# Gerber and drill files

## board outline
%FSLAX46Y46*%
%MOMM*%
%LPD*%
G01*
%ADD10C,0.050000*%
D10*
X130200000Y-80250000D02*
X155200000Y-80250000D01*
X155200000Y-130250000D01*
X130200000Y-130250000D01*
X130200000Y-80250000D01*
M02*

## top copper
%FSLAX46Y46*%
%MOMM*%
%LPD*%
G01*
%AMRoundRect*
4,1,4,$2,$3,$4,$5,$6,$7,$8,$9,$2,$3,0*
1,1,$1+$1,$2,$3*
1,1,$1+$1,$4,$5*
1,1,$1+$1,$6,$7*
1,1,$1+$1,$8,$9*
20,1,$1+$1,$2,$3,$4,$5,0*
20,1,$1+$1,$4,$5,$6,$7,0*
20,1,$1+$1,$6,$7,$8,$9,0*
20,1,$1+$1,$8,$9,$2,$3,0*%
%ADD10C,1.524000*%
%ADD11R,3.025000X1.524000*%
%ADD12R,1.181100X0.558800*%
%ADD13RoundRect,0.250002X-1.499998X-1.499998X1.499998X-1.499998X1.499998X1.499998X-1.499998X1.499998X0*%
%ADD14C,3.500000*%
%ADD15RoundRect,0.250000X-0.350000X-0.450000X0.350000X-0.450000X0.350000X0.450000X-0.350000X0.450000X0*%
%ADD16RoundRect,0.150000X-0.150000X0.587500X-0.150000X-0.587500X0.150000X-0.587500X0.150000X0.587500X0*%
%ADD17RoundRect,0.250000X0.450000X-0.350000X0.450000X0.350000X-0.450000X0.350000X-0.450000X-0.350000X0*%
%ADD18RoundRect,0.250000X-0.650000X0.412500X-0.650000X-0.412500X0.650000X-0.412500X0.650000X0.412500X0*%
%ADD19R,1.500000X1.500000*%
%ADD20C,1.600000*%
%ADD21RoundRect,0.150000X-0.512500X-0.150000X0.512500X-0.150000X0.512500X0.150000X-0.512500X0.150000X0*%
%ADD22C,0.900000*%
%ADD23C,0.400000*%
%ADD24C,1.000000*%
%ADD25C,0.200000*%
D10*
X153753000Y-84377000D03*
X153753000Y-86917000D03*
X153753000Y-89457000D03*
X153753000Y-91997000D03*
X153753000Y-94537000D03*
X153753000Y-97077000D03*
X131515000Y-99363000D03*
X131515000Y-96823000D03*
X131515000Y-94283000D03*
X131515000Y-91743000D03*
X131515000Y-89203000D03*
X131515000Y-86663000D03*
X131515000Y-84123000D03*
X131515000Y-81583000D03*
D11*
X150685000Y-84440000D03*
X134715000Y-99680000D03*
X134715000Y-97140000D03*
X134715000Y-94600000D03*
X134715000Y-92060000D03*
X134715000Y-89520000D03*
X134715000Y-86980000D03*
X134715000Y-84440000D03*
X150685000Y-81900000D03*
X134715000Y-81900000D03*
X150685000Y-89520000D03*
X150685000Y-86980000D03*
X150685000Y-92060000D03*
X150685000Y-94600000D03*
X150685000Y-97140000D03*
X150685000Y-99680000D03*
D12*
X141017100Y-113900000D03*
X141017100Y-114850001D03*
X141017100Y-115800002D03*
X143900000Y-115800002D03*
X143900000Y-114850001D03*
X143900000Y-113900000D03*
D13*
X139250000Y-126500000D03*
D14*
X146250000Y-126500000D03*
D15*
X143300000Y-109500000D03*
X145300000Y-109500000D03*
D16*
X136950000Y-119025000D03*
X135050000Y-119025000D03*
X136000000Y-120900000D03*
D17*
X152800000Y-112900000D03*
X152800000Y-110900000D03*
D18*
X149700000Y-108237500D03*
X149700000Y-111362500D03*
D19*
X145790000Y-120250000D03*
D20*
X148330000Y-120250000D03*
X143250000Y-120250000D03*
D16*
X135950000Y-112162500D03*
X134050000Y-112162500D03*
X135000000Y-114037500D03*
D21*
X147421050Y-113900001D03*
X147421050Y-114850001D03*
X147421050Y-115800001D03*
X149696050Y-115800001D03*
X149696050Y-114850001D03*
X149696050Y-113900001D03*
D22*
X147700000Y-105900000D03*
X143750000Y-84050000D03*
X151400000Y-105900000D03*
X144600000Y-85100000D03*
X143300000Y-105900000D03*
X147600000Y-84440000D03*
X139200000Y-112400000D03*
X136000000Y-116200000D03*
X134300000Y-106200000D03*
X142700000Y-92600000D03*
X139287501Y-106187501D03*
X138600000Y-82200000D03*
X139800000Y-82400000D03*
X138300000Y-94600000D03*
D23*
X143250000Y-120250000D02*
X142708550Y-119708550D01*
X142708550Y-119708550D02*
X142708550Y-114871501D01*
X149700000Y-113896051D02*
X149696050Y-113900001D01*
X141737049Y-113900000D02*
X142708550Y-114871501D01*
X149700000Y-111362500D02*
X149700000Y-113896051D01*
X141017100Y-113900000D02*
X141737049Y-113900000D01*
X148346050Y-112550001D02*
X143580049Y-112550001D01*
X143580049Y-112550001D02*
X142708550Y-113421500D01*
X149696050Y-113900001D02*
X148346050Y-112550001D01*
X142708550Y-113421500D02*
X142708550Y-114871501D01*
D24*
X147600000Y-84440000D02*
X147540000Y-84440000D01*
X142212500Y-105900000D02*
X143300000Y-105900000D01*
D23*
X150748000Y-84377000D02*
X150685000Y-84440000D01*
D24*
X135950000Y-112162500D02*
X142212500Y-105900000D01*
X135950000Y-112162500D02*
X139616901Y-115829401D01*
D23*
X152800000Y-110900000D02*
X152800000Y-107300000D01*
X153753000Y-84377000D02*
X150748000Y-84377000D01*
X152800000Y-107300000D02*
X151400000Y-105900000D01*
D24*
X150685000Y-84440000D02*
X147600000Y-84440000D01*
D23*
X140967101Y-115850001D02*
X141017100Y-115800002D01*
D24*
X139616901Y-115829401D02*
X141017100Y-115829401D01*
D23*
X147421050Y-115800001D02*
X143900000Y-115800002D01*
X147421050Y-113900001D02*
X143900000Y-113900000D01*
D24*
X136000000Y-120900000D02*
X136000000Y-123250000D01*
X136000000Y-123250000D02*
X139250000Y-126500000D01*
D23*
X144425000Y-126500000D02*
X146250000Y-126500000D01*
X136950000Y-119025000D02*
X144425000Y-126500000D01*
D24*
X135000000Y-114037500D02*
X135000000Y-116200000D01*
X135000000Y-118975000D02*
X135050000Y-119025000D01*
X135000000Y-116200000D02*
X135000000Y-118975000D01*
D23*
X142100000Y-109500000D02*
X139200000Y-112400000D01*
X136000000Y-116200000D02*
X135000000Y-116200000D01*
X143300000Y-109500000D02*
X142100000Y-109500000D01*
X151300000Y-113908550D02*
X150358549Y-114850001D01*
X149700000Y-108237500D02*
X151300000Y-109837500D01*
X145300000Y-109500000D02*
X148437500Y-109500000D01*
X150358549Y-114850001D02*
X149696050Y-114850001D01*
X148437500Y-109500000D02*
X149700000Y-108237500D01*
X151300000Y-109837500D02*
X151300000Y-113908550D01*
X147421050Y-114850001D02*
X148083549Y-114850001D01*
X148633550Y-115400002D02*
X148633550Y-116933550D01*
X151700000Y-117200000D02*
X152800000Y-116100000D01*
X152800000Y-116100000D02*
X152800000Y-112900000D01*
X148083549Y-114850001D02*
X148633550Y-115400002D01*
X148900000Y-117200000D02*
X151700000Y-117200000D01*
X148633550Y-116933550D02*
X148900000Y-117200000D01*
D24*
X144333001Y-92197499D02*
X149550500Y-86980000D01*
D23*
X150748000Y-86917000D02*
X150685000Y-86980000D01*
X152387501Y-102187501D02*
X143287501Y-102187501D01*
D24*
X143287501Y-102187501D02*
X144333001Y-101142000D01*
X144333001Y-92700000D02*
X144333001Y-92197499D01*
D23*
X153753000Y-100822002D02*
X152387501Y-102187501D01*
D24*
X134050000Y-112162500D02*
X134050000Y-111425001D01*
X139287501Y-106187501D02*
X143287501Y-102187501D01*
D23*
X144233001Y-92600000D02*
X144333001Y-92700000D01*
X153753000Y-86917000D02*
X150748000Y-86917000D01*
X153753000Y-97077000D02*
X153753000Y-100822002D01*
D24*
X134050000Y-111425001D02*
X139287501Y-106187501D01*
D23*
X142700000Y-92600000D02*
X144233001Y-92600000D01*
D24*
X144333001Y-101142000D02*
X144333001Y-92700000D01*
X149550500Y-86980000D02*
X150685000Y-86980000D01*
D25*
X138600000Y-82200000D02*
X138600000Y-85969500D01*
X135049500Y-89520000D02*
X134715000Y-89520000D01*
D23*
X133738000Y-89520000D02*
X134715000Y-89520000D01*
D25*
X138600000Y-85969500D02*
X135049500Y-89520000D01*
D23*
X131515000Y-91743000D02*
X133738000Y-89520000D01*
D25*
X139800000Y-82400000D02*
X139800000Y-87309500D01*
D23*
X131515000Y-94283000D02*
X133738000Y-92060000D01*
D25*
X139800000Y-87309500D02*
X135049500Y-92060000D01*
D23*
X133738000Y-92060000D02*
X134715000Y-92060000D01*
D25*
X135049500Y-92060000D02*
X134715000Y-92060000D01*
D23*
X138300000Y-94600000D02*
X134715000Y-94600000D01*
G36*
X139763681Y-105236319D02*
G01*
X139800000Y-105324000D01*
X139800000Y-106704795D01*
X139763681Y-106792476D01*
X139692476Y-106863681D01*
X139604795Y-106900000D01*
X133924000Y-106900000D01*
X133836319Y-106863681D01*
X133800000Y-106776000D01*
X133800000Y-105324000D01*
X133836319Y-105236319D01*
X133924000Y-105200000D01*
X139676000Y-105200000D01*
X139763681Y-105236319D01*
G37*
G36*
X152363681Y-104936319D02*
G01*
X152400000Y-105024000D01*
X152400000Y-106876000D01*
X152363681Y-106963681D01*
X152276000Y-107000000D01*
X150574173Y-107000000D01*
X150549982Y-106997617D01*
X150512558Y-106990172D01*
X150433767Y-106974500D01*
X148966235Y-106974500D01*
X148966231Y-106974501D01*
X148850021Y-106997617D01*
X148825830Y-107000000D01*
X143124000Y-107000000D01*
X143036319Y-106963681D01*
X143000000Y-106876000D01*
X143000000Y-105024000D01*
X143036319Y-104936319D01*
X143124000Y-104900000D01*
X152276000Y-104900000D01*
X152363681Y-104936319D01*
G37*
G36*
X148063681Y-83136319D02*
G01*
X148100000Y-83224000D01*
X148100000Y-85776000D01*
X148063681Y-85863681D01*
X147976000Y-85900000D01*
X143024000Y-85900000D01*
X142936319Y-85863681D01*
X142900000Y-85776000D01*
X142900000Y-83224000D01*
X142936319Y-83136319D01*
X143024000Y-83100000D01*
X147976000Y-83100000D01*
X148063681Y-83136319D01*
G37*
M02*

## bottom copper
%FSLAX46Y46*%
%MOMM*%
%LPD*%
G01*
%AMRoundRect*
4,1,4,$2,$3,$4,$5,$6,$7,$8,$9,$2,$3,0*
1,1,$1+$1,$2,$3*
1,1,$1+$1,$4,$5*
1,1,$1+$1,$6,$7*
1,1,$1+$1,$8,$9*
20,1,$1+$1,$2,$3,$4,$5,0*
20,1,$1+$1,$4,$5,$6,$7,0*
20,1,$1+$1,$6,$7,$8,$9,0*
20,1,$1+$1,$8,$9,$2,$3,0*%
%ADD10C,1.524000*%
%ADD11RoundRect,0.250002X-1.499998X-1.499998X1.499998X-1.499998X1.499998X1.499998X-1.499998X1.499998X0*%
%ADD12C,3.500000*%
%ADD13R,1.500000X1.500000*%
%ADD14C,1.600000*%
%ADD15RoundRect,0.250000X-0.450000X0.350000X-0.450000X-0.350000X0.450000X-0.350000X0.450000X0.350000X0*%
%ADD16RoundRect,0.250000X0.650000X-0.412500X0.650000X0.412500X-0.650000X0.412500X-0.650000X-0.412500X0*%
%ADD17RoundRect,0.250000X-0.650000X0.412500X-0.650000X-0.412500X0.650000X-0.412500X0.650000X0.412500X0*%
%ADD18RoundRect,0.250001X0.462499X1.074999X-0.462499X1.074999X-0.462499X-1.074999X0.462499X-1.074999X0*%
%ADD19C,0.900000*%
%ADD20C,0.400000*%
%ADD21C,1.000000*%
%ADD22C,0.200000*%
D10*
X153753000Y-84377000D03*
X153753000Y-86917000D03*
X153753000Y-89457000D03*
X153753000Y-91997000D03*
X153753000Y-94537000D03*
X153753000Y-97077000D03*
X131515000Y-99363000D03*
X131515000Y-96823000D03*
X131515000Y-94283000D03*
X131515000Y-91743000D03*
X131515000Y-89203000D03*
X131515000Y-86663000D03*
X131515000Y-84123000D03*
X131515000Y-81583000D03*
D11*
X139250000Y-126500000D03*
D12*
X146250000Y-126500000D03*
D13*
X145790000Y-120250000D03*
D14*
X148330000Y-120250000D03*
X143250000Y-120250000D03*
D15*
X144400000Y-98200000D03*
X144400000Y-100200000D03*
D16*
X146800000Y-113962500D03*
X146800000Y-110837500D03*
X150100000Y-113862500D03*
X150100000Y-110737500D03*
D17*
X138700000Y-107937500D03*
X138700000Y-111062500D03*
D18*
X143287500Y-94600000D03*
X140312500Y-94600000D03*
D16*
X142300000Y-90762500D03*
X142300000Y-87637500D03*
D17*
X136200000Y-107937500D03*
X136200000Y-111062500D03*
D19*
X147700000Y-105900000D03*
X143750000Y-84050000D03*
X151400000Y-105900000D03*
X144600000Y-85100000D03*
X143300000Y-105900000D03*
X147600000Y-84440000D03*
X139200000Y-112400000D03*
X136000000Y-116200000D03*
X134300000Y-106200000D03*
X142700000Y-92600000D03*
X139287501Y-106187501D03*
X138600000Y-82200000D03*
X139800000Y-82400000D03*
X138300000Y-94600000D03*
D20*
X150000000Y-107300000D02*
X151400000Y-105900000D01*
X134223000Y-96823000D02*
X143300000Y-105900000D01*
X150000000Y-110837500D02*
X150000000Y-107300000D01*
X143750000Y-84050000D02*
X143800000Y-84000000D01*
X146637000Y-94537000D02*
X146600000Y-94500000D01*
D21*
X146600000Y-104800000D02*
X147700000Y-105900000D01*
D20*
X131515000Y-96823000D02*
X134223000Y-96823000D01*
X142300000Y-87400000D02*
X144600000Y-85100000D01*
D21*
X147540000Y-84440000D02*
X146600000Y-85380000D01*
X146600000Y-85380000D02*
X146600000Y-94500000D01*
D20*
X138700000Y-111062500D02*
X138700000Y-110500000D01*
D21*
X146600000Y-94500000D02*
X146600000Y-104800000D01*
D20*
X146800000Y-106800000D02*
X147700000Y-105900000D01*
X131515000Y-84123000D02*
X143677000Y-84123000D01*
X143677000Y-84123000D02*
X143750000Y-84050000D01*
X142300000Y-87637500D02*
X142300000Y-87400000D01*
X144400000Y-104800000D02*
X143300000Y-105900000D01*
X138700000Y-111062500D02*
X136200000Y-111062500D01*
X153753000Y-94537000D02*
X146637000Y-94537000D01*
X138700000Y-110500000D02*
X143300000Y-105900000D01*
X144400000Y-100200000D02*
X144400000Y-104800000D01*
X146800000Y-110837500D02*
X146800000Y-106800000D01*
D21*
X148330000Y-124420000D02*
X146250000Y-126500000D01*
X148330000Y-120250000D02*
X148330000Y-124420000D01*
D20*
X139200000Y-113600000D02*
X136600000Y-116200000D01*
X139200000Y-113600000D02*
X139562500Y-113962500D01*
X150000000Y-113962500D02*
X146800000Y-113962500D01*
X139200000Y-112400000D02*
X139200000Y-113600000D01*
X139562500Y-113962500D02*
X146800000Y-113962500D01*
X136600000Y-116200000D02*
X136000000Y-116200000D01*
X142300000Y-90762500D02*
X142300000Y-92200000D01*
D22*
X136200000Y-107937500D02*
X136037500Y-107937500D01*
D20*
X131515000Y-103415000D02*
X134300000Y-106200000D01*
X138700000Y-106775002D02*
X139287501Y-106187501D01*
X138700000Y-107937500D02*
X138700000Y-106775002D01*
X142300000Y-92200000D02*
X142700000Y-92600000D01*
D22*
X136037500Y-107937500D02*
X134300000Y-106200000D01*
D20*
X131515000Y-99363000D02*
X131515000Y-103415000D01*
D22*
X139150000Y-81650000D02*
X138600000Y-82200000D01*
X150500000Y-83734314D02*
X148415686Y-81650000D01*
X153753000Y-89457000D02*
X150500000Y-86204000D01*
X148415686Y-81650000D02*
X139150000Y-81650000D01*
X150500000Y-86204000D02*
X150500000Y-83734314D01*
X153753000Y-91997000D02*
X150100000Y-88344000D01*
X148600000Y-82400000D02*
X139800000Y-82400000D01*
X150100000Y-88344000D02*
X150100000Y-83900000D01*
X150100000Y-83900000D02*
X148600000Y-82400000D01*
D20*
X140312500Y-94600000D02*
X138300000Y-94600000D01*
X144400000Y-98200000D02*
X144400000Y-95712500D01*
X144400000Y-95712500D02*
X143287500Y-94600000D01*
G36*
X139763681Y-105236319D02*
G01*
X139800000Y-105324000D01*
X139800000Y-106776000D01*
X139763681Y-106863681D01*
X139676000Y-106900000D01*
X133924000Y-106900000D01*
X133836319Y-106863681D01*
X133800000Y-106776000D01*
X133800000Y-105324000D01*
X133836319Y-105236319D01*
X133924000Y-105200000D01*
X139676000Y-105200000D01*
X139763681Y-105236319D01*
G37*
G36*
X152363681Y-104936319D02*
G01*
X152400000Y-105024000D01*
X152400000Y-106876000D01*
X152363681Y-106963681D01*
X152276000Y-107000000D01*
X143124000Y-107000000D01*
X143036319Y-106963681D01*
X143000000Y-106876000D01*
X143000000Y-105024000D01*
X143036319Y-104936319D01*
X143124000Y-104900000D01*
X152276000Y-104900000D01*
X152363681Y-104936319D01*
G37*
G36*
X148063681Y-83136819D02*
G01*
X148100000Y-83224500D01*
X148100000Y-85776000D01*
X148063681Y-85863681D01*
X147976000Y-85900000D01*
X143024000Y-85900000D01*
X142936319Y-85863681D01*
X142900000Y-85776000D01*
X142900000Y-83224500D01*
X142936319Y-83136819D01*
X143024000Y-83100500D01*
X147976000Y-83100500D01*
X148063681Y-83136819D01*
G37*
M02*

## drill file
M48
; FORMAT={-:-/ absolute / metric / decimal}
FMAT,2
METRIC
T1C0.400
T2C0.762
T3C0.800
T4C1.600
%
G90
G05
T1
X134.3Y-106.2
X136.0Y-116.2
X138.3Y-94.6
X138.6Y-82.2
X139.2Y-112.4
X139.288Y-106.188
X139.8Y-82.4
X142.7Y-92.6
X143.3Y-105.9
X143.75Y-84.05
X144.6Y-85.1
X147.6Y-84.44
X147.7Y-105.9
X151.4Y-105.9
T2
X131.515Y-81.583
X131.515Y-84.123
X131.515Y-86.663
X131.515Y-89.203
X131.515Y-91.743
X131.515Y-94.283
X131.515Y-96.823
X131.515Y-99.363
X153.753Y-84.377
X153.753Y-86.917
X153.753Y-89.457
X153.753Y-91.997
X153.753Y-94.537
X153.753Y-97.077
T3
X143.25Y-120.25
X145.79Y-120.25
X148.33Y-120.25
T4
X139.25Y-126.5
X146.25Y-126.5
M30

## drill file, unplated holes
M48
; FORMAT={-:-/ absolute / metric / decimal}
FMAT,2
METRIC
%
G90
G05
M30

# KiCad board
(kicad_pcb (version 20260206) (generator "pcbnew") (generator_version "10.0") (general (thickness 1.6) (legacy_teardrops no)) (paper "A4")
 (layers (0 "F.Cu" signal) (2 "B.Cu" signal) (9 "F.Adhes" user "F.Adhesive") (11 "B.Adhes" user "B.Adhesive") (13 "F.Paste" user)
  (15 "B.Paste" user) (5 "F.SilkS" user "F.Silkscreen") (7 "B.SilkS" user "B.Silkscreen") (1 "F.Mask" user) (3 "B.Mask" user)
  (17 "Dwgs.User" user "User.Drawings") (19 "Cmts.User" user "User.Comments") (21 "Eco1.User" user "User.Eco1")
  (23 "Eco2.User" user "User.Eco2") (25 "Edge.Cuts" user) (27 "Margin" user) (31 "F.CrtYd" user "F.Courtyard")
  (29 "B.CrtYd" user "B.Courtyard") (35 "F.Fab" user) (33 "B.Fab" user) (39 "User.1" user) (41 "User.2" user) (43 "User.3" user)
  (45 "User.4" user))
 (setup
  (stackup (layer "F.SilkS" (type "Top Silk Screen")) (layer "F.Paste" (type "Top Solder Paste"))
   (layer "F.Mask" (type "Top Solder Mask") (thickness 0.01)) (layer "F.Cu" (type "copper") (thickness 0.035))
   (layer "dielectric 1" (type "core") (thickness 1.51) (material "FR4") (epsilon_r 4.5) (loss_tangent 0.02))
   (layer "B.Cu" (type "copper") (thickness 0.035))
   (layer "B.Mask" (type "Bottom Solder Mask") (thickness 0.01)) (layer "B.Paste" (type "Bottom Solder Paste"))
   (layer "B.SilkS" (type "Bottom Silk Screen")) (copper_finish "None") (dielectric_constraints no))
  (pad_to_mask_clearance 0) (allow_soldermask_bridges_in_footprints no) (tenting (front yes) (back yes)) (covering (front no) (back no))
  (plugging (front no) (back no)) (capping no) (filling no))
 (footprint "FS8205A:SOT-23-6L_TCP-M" (layer "F.Cu") (at 142.45855 114.850001)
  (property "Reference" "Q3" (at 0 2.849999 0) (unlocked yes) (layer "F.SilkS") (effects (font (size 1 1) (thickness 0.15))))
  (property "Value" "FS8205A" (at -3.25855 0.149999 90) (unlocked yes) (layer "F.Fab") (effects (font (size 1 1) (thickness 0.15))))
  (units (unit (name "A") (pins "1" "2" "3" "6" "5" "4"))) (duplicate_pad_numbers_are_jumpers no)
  (pad "1" smd rect (at -1.44145 -0.950001) (size 1.1811 0.5588) (layers "F.Cu" "F.Mask" "F.Paste") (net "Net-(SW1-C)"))
  (pad "2" smd rect (at -1.44145 0) (size 1.1811 0.5588) (layers "F.Cu" "F.Mask" "F.Paste") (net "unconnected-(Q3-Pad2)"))
  (pad "3" smd rect (at -1.44145 0.950001) (size 1.1811 0.5588) (layers "F.Cu" "F.Mask" "F.Paste") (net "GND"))
  (pad "4" smd rect (at 1.44145 0.950001) (size 1.1811 0.5588) (layers "F.Cu" "F.Mask" "F.Paste") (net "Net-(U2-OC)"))
  (pad "5" smd rect (at 1.44145 0) (size 1.1811 0.5588) (layers "F.Cu" "F.Mask" "F.Paste") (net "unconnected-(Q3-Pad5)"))
  (pad "6" smd rect (at 1.44145 -0.950001) (size 1.1811 0.5588) (layers "F.Cu" "F.Mask" "F.Paste") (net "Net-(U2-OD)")))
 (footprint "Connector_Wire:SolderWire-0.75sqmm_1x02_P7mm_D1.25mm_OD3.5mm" (layer "F.Cu") (at 139.25 126.5)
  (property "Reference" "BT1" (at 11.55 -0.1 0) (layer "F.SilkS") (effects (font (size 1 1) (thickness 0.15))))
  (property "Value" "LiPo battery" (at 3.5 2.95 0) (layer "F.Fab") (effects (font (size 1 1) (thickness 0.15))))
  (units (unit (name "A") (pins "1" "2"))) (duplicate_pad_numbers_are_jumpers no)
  (pad "1" thru_hole roundrect (at 0 0) (size 3.5 3.5) (drill 1.6) (layers "*.Cu" "*.Mask") (remove_unused_layers no)
   (roundrect_rratio 0.071429) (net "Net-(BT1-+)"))
  (pad "2" thru_hole circle (at 7 0) (size 3.5 3.5) (drill 1.6) (layers "*.Cu" "*.Mask") (remove_unused_layers no) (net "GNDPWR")))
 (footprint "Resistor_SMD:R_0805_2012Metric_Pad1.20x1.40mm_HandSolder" (layer "F.Cu") (at 144.3 109.5)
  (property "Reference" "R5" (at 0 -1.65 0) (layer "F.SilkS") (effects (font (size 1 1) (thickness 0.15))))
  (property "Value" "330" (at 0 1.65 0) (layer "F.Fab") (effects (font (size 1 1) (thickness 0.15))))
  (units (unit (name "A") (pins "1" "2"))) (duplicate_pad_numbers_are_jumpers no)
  (pad "1" smd roundrect (at -1 0) (size 1.2 1.4) (layers "F.Cu" "F.Mask" "F.Paste") (roundrect_rratio 0.208333) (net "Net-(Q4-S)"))
  (pad "2" smd roundrect (at 1 0) (size 1.2 1.4) (layers "F.Cu" "F.Mask" "F.Paste") (roundrect_rratio 0.208333) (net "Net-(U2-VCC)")))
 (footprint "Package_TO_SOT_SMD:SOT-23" (layer "F.Cu") (at 136 119.9625 -90)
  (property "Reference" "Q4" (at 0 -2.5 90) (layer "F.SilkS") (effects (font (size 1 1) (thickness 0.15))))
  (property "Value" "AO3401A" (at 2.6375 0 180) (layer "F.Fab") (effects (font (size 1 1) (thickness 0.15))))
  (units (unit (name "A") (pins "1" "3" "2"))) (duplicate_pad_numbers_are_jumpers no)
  (pad "1" smd roundrect (at -0.9375 -0.95 270) (size 1.475 0.6) (layers "F.Cu" "F.Mask" "F.Paste") (roundrect_rratio 0.25) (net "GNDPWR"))
  (pad "2" smd roundrect (at -0.9375 0.95 270) (size 1.475 0.6) (layers "F.Cu" "F.Mask" "F.Paste") (roundrect_rratio 0.25)
   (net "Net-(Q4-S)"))
  (pad "3" smd roundrect (at 0.9375 0 270) (size 1.475 0.6) (layers "F.Cu" "F.Mask" "F.Paste") (roundrect_rratio 0.25) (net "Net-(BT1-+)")))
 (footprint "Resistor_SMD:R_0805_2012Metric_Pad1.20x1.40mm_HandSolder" (layer "F.Cu") (at 152.8 111.9 90)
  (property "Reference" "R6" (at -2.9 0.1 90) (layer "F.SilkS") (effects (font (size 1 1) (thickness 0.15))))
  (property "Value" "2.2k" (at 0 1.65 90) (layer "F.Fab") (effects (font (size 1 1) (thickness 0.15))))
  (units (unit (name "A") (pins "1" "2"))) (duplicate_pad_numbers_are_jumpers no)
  (pad "1" smd roundrect (at -1 0 90) (size 1.2 1.4) (layers "F.Cu" "F.Mask" "F.Paste") (roundrect_rratio 0.208333) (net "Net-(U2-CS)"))
  (pad "2" smd roundrect (at 1 0 90) (size 1.2 1.4) (layers "F.Cu" "F.Mask" "F.Paste") (roundrect_rratio 0.208333) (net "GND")))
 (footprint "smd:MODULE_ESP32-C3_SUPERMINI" (layer "F.Cu") (at 142.7 91.8)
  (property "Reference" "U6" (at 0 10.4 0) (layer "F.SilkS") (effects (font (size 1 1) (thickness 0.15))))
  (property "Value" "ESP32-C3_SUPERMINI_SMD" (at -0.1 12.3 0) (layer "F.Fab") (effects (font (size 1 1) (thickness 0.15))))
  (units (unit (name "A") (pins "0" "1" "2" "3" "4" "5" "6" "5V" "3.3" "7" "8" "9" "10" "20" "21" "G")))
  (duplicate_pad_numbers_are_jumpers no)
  (pad "0" smd rect (at 7.985 7.88) (size 3.025 1.524) (layers "F.Cu" "F.Mask" "F.Paste") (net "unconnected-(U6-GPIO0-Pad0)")
   (solder_mask_margin 0.102))
  (pad "1" smd rect (at 7.985 5.34) (size 3.025 1.524) (layers "F.Cu" "F.Mask" "F.Paste") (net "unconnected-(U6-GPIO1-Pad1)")
   (solder_mask_margin 0.102))
  (pad "2" smd rect (at 7.985 2.8) (size 3.025 1.524) (layers "F.Cu" "F.Mask" "F.Paste") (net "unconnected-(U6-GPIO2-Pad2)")
   (solder_mask_margin 0.102))
  (pad "3" smd rect (at 7.985 0.26) (size 3.025 1.524) (layers "F.Cu" "F.Mask" "F.Paste") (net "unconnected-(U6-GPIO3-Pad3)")
   (solder_mask_margin 0.102))
  (pad "3.3" smd rect (at 7.985 -4.82) (size 3.025 1.524) (layers "F.Cu" "F.Mask" "F.Paste") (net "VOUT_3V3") (solder_mask_margin 0.102))
  (pad "4" smd rect (at 7.985 -2.28) (size 3.025 1.524) (layers "F.Cu" "F.Mask" "F.Paste") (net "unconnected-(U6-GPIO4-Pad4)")
   (solder_mask_margin 0.102))
  (pad "5" smd rect (at -7.985 -9.9) (size 3.025 1.524) (layers "F.Cu" "F.Mask" "F.Paste") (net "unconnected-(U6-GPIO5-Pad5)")
   (solder_mask_margin 0.102))
  (pad "5V" smd rect (at 7.985 -9.9) (size 3.025 1.524) (layers "F.Cu" "F.Mask" "F.Paste") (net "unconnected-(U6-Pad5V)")
   (solder_mask_margin 0.102))
  (pad "6" smd rect (at -7.985 -7.36) (size 3.025 1.524) (layers "F.Cu" "F.Mask" "F.Paste") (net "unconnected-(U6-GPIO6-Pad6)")
   (solder_mask_margin 0.102))
  (pad "7" smd rect (at -7.985 -4.82) (size 3.025 1.524) (layers "F.Cu" "F.Mask" "F.Paste") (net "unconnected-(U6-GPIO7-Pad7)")
   (solder_mask_margin 0.102))
  (pad "8" smd rect (at -7.985 -2.28) (size 3.025 1.524) (layers "F.Cu" "F.Mask" "F.Paste") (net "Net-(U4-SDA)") (solder_mask_margin 0.102))
  (pad "9" smd rect (at -7.985 0.26) (size 3.025 1.524) (layers "F.Cu" "F.Mask" "F.Paste") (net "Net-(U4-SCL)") (solder_mask_margin 0.102))
  (pad "10" smd rect (at -7.985 2.8) (size 3.025 1.524) (layers "F.Cu" "F.Mask" "F.Paste") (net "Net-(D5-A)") (solder_mask_margin 0.102))
  (pad "20" smd rect (at -7.985 5.34) (size 3.025 1.524) (layers "F.Cu" "F.Mask" "F.Paste") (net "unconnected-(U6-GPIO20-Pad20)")
   (solder_mask_margin 0.102))
  (pad "21" smd rect (at -7.985 7.88) (size 3.025 1.524) (layers "F.Cu" "F.Mask" "F.Paste") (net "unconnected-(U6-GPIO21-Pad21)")
   (solder_mask_margin 0.102))
  (pad "G" smd rect (at 7.985 -7.36) (size 3.025 1.524) (layers "F.Cu" "F.Mask" "F.Paste") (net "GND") (solder_mask_margin 0.102)))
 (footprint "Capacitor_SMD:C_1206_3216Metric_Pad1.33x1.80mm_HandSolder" (layer "F.Cu") (at 149.7 109.8 -90)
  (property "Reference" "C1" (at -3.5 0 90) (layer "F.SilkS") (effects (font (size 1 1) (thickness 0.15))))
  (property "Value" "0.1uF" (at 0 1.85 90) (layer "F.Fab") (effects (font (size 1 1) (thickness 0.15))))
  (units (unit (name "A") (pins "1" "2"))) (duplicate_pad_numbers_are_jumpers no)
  (pad "1" smd roundrect (at -1.5625 0 270) (size 1.325 1.8) (layers "F.Cu" "F.Mask" "F.Paste") (roundrect_rratio 0.188679)
   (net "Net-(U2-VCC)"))
  (pad "2" smd roundrect (at 1.5625 0 270) (size 1.325 1.8) (layers "F.Cu" "F.Mask" "F.Paste") (roundrect_rratio 0.188679)
   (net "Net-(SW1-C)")))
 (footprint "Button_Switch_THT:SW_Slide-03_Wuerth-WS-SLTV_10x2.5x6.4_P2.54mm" (layer "F.Cu") (at 145.79 120.25 180)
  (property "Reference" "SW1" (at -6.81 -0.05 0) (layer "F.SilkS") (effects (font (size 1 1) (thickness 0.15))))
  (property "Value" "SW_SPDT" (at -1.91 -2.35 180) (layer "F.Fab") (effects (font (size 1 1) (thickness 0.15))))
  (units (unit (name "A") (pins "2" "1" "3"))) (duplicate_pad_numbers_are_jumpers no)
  (pad "1" thru_hole rect (at 0 0 180) (size 1.5 1.5) (drill 0.8) (layers "*.Cu" "*.Mask") (remove_unused_layers no)
   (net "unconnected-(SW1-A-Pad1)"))
  (pad "2" thru_hole circle (at -2.54 0 180) (size 1.6 1.6) (drill 0.8) (layers "*.Cu" "*.Mask") (remove_unused_layers no) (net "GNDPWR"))
  (pad "3" thru_hole circle (at 2.54 0 180) (size 1.6 1.6) (drill 0.8) (layers "*.Cu" "*.Mask") (remove_unused_layers no)
   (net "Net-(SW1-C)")))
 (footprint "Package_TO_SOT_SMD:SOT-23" (layer "F.Cu") (at 135 113.1 -90)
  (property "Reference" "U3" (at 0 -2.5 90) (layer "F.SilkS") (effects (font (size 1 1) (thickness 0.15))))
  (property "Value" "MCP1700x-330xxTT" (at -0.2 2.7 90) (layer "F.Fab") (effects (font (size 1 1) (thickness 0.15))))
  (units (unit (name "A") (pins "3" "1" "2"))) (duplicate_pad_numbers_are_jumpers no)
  (pad "1" smd roundrect (at -0.9375 -0.95 270) (size 1.475 0.6) (layers "F.Cu" "F.Mask" "F.Paste") (roundrect_rratio 0.25) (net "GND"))
  (pad "2" smd roundrect (at -0.9375 0.95 270) (size 1.475 0.6) (layers "F.Cu" "F.Mask" "F.Paste") (roundrect_rratio 0.25) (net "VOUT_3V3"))
  (pad "3" smd roundrect (at 0.9375 0 270) (size 1.475 0.6) (layers "F.Cu" "F.Mask" "F.Paste") (roundrect_rratio 0.25) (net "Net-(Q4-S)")))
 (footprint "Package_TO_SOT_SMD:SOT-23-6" (layer "F.Cu") (at 148.55855 114.850001)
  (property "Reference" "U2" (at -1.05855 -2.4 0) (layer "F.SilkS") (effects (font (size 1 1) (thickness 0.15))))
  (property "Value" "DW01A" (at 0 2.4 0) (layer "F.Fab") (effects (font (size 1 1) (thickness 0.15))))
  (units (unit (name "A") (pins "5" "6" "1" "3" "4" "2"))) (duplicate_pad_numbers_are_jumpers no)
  (pad "1" smd roundrect (at -1.1375 -0.95) (size 1.325 0.6) (layers "F.Cu" "F.Mask" "F.Paste") (roundrect_rratio 0.25) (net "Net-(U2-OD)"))
  (pad "2" smd roundrect (at -1.1375 0) (size 1.325 0.6) (layers "F.Cu" "F.Mask" "F.Paste") (roundrect_rratio 0.25) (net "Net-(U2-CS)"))
  (pad "3" smd roundrect (at -1.1375 0.95) (size 1.325 0.6) (layers "F.Cu" "F.Mask" "F.Paste") (roundrect_rratio 0.25) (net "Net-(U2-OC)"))
  (pad "4" smd roundrect (at 1.1375 0.95) (size 1.325 0.6) (layers "F.Cu" "F.Mask" "F.Paste") (roundrect_rratio 0.25)
   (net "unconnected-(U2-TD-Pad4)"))
  (pad "5" smd roundrect (at 1.1375 0) (size 1.325 0.6) (layers "F.Cu" "F.Mask" "F.Paste") (roundrect_rratio 0.25) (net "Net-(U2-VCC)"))
  (pad "6" smd roundrect (at 1.1375 -0.95) (size 1.325 0.6) (layers "F.Cu" "F.Mask" "F.Paste") (roundrect_rratio 0.25) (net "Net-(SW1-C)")))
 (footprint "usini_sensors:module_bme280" (layer "F.Cu") (at 148.673 84.631 180)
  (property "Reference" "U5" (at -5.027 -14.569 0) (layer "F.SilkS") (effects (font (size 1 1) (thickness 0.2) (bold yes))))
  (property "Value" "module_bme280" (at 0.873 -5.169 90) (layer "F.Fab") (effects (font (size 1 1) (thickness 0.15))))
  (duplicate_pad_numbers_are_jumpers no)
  (pad "1" thru_hole circle (at -5.08 -12.446 180) (size 1.524 1.524) (drill 0.762) (layers "*.Cu" "*.Mask") (remove_unused_layers no)
   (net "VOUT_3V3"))
  (pad "2" thru_hole circle (at -5.08 -9.906 180) (size 1.524 1.524) (drill 0.762) (layers "*.Cu" "*.Mask") (remove_unused_layers no)
   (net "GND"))
  (pad "3" thru_hole circle (at -5.08 -7.366 180) (size 1.524 1.524) (drill 0.762) (layers "*.Cu" "*.Mask") (remove_unused_layers no)
   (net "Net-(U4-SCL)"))
  (pad "4" thru_hole circle (at -5.08 -4.826 180) (size 1.524 1.524) (drill 0.762) (layers "*.Cu" "*.Mask") (remove_unused_layers no)
   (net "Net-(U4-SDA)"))
  (pad "5" thru_hole circle (at -5.08 -2.286 180) (size 1.524 1.524) (drill 0.762) (layers "*.Cu" "*.Mask") (remove_unused_layers no)
   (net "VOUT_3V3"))
  (pad "6" thru_hole circle (at -5.08 0.254 180) (size 1.524 1.524) (drill 0.762) (layers "*.Cu" "*.Mask") (remove_unused_layers no)
   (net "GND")))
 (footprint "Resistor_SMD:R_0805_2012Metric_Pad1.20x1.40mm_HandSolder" (layer "B.Cu") (at 144.4 99.2 -90)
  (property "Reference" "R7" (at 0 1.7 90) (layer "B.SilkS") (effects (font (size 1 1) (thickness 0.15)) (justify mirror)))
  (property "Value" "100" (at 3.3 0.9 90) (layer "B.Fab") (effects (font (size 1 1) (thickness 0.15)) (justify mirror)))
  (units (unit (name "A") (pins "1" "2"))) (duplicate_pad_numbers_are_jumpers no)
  (pad "1" smd roundrect (at -1 0 270) (size 1.2 1.4) (layers "B.Cu" "B.Mask" "B.Paste") (roundrect_rratio 0.208333) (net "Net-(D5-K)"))
  (pad "2" smd roundrect (at 1 0 270) (size 1.2 1.4) (layers "B.Cu" "B.Mask" "B.Paste") (roundrect_rratio 0.208333) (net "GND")))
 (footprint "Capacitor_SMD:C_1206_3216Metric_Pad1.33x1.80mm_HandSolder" (layer "B.Cu") (at 146.8 112.4 90)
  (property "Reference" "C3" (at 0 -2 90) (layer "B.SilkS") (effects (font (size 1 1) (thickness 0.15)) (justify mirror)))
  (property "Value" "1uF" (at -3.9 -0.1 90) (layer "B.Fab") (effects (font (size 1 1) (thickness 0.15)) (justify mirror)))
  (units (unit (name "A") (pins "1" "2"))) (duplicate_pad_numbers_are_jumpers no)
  (pad "1" smd roundrect (at -1.5625 0 90) (size 1.325 1.8) (layers "B.Cu" "B.Mask" "B.Paste") (roundrect_rratio 0.188679)
   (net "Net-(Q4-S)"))
  (pad "2" smd roundrect (at 1.5625 0 90) (size 1.325 1.8) (layers "B.Cu" "B.Mask" "B.Paste") (roundrect_rratio 0.188679) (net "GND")))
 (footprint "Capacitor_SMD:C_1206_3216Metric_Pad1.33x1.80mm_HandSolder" (layer "B.Cu") (at 150.1 112.3 90)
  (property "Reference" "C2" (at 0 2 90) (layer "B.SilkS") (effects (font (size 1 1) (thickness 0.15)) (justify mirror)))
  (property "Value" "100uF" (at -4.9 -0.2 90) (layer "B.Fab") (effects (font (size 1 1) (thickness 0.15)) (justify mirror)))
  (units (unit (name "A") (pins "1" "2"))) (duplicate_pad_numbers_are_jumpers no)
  (pad "1" smd roundrect (at -1.5625 0 90) (size 1.325 1.8) (layers "B.Cu" "B.Mask" "B.Paste") (roundrect_rratio 0.188679)
   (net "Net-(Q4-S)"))
  (pad "2" smd roundrect (at 1.5625 0 90) (size 1.325 1.8) (layers "B.Cu" "B.Mask" "B.Paste") (roundrect_rratio 0.188679) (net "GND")))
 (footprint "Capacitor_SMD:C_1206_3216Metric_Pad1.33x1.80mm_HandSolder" (layer "B.Cu") (at 138.7 109.5 -90)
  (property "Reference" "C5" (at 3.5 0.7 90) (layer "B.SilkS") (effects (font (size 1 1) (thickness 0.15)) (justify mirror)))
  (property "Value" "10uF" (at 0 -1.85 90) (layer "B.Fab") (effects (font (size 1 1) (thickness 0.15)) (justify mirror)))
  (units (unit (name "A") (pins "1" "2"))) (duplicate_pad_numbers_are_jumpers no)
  (pad "1" smd roundrect (at -1.5625 0 270) (size 1.325 1.8) (layers "B.Cu" "B.Mask" "B.Paste") (roundrect_rratio 0.188679) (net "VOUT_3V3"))
  (pad "2" smd roundrect (at 1.5625 0 270) (size 1.325 1.8) (layers "B.Cu" "B.Mask" "B.Paste") (roundrect_rratio 0.188679) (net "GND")))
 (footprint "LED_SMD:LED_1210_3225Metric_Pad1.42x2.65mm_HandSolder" (layer "B.Cu") (at 141.8 94.6 180)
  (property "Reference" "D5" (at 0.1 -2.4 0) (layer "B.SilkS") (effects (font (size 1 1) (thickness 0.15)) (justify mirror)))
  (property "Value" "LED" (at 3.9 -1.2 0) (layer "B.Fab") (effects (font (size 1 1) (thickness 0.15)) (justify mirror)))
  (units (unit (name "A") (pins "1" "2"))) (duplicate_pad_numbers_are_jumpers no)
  (pad "1" smd roundrect (at -1.4875 0 180) (size 1.425 2.65) (layers "B.Cu" "B.Mask" "B.Paste") (roundrect_rratio 0.175439)
   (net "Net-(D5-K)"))
  (pad "2" smd roundrect (at 1.4875 0 180) (size 1.425 2.65) (layers "B.Cu" "B.Mask" "B.Paste") (roundrect_rratio 0.175439)
   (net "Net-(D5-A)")))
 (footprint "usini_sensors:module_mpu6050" (layer "B.Cu") (at 131.515 81.583)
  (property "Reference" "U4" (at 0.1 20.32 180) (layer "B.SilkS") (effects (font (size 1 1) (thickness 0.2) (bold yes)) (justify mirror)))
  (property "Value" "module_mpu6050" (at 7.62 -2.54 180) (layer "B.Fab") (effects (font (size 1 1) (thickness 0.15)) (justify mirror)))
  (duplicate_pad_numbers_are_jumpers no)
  (pad "1" thru_hole circle (at 0 17.78) (size 1.524 1.524) (drill 0.762) (layers "*.Cu" "*.Mask") (remove_unused_layers no)
   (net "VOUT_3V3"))
  (pad "2" thru_hole circle (at 0 15.24) (size 1.524 1.524) (drill 0.762) (layers "*.Cu" "*.Mask") (remove_unused_layers no) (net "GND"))
  (pad "3" thru_hole circle (at 0 12.7) (size 1.524 1.524) (drill 0.762) (layers "*.Cu" "*.Mask") (remove_unused_layers no)
   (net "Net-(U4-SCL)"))
  (pad "4" thru_hole circle (at 0 10.16) (size 1.524 1.524) (drill 0.762) (layers "*.Cu" "*.Mask") (remove_unused_layers no)
   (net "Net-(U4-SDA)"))
  (pad "5" thru_hole circle (at 0 7.62) (size 1.524 1.524) (drill 0.762) (layers "*.Cu" "*.Mask") (remove_unused_layers no)
   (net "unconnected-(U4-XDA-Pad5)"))
  (pad "6" thru_hole circle (at 0 5.08) (size 1.524 1.524) (drill 0.762) (layers "*.Cu" "*.Mask") (remove_unused_layers no)
   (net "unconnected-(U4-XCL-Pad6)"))
  (pad "7" thru_hole circle (at 0 2.54) (size 1.524 1.524) (drill 0.762) (layers "*.Cu" "*.Mask") (remove_unused_layers no) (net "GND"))
  (pad "8" thru_hole circle (at 0 0) (size 1.524 1.524) (drill 0.762) (layers "*.Cu" "*.Mask") (remove_unused_layers no)
   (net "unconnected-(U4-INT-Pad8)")))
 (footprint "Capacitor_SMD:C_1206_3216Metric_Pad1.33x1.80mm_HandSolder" (layer "B.Cu") (at 142.3 89.2 90)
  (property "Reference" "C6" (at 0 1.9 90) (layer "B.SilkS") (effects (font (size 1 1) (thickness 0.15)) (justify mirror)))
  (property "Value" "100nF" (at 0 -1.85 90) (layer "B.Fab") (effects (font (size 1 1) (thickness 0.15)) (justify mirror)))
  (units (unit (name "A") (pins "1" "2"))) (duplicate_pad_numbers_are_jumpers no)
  (pad "1" smd roundrect (at -1.5625 0 90) (size 1.325 1.8) (layers "B.Cu" "B.Mask" "B.Paste") (roundrect_rratio 0.188679) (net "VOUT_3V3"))
  (pad "2" smd roundrect (at 1.5625 0 90) (size 1.325 1.8) (layers "B.Cu" "B.Mask" "B.Paste") (roundrect_rratio 0.188679) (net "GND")))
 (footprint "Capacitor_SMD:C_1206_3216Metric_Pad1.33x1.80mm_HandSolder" (layer "B.Cu") (at 136.2 109.5 -90)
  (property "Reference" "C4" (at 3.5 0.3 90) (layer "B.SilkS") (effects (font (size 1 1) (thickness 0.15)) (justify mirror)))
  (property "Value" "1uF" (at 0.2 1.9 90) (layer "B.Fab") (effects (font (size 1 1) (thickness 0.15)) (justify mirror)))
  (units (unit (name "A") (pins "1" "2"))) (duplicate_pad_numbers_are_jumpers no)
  (pad "1" smd roundrect (at -1.5625 0 270) (size 1.325 1.8) (layers "B.Cu" "B.Mask" "B.Paste") (roundrect_rratio 0.188679) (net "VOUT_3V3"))
  (pad "2" smd roundrect (at 1.5625 0 270) (size 1.325 1.8) (layers "B.Cu" "B.Mask" "B.Paste") (roundrect_rratio 0.188679) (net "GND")))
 (gr_rect (start 130.2 80.25) (end 155.2 130.25) (stroke (width 0.05) (type solid)) (fill no) (layer "Edge.Cuts"))
 (segment (start 143.25 120.25) (end 142.70855 119.70855) (width 0.4) (layer "F.Cu") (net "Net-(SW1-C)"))
 (segment (start 142.70855 119.70855) (end 142.70855 114.871501) (width 0.4) (layer "F.Cu") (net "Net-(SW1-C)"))
 (segment (start 149.7 113.896051) (end 149.69605 113.900001) (width 0.4) (layer "F.Cu") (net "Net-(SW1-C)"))
 (segment (start 141.737049 113.9) (end 142.70855 114.871501) (width 0.4) (layer "F.Cu") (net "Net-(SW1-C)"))
 (segment (start 149.7 111.3625) (end 149.7 113.896051) (width 0.4) (layer "F.Cu") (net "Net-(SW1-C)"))
 (segment (start 141.0171 113.9) (end 141.737049 113.9) (width 0.4) (layer "F.Cu") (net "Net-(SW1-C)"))
 (segment (start 148.34605 112.550001) (end 143.580049 112.550001) (width 0.4) (layer "F.Cu") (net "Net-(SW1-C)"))
 (segment (start 143.580049 112.550001) (end 142.70855 113.4215) (width 0.4) (layer "F.Cu") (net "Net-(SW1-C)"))
 (segment (start 149.69605 113.900001) (end 148.34605 112.550001) (width 0.4) (layer "F.Cu") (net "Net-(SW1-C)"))
 (segment (start 142.70855 113.4215) (end 142.70855 114.871501) (width 0.4) (layer "F.Cu") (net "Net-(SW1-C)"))
 (segment (start 147.6 84.44) (end 147.54 84.44) (width 1) (layer "F.Cu") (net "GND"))
 (segment (start 142.2125 105.9) (end 143.3 105.9) (width 1) (layer "F.Cu") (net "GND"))
 (segment (start 150.748 84.377) (end 150.685 84.44) (width 0.4) (layer "F.Cu") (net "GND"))
 (segment (start 135.95 112.1625) (end 142.2125 105.9) (width 1) (layer "F.Cu") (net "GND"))
 (segment (start 135.95 112.1625) (end 139.616901 115.829401) (width 1) (layer "F.Cu") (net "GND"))
 (segment (start 152.8 110.9) (end 152.8 107.3) (width 0.4) (layer "F.Cu") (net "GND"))
 (segment (start 153.753 84.377) (end 150.748 84.377) (width 0.4) (layer "F.Cu") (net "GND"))
 (segment (start 152.8 107.3) (end 151.4 105.9) (width 0.4) (layer "F.Cu") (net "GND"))
 (segment (start 150.685 84.44) (end 147.6 84.44) (width 1) (layer "F.Cu") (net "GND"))
 (segment (start 140.967101 115.850001) (end 141.0171 115.800002) (width 0.4) (layer "F.Cu") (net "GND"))
 (segment (start 139.616901 115.829401) (end 141.0171 115.829401) (width 1) (layer "F.Cu") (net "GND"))
 (via (at 147.7 105.9) (size 0.9) (drill 0.4) (layers "F.Cu" "B.Cu") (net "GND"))
 (via (at 143.75 84.05) (size 0.9) (drill 0.4) (layers "F.Cu" "B.Cu") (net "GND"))
 (via (at 151.4 105.9) (size 0.9) (drill 0.4) (layers "F.Cu" "B.Cu") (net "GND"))
 (via (at 144.6 85.1) (size 0.9) (drill 0.4) (layers "F.Cu" "B.Cu") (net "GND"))
 (via (at 143.3 105.9) (size 0.9) (drill 0.4) (layers "F.Cu" "B.Cu") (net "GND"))
 (via (at 147.6 84.44) (size 0.9) (drill 0.4) (layers "F.Cu" "B.Cu") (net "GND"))
 (segment (start 150 107.3) (end 151.4 105.9) (width 0.4) (layer "B.Cu") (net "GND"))
 (segment (start 134.223 96.823) (end 143.3 105.9) (width 0.4) (layer "B.Cu") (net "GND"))
 (segment (start 150 110.8375) (end 150 107.3) (width 0.4) (layer "B.Cu") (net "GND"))
 (segment (start 143.75 84.05) (end 143.8 84) (width 0.4) (layer "B.Cu") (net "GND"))
 (segment (start 146.637 94.537) (end 146.6 94.5) (width 0.4) (layer "B.Cu") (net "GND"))
 (segment (start 146.6 104.8) (end 147.7 105.9) (width 1) (layer "B.Cu") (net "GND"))
 (segment (start 131.515 96.823) (end 134.223 96.823) (width 0.4) (layer "B.Cu") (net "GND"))
 (segment (start 142.3 87.4) (end 144.6 85.1) (width 0.4) (layer "B.Cu") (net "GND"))
 (segment (start 147.54 84.44) (end 146.6 85.38) (width 1) (layer "B.Cu") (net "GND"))
 (segment (start 146.6 85.38) (end 146.6 94.5) (width 1) (layer "B.Cu") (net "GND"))
 (segment (start 138.7 111.0625) (end 138.7 110.5) (width 0.4) (layer "B.Cu") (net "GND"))
 (segment (start 146.6 94.5) (end 146.6 104.8) (width 1) (layer "B.Cu") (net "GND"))
 (segment (start 146.8 106.8) (end 147.7 105.9) (width 0.4) (layer "B.Cu") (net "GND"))
 (segment (start 131.515 84.123) (end 143.677 84.123) (width 0.4) (layer "B.Cu") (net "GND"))
 (segment (start 143.677 84.123) (end 143.75 84.05) (width 0.4) (layer "B.Cu") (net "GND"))
 (segment (start 142.3 87.6375) (end 142.3 87.4) (width 0.4) (layer "B.Cu") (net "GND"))
 (segment (start 144.4 104.8) (end 143.3 105.9) (width 0.4) (layer "B.Cu") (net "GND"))
 (segment (start 138.7 111.0625) (end 136.2 111.0625) (width 0.4) (layer "B.Cu") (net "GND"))
 (segment (start 153.753 94.537) (end 146.637 94.537) (width 0.4) (layer "B.Cu") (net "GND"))
 (segment (start 138.7 110.5) (end 143.3 105.9) (width 0.4) (layer "B.Cu") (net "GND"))
 (segment (start 144.4 100.2) (end 144.4 104.8) (width 0.4) (layer "B.Cu") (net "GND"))
 (segment (start 146.8 110.8375) (end 146.8 106.8) (width 0.4) (layer "B.Cu") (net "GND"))
 (segment (start 147.42105 115.800001) (end 143.9 115.800002) (width 0.4) (layer "F.Cu") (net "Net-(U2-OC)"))
 (segment (start 147.42105 113.900001) (end 143.9 113.9) (width 0.4) (layer "F.Cu") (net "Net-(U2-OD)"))
 (segment (start 136 120.9) (end 136 123.25) (width 1) (layer "F.Cu") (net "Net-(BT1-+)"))
 (segment (start 136 123.25) (end 139.25 126.5) (width 1) (layer "F.Cu") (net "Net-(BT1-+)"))
 (segment (start 144.425 126.5) (end 146.25 126.5) (width 0.4) (layer "F.Cu") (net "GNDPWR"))
 (segment (start 136.95 119.025) (end 144.425 126.5) (width 0.4) (layer "F.Cu") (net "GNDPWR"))
 (segment (start 148.33 124.42) (end 146.25 126.5) (width 1) (layer "B.Cu") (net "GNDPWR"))
 (segment (start 148.33 120.25) (end 148.33 124.42) (width 1) (layer "B.Cu") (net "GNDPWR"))
 (segment (start 135 114.0375) (end 135 116.2) (width 1) (layer "F.Cu") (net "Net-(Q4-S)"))
 (segment (start 135 118.975) (end 135.05 119.025) (width 1) (layer "F.Cu") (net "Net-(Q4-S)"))
 (segment (start 135 116.2) (end 135 118.975) (width 1) (layer "F.Cu") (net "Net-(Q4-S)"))
 (segment (start 142.1 109.5) (end 139.2 112.4) (width 0.4) (layer "F.Cu") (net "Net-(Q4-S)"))
 (segment (start 136 116.2) (end 135 116.2) (width 0.4) (layer "F.Cu") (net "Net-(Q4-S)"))
 (segment (start 143.3 109.5) (end 142.1 109.5) (width 0.4) (layer "F.Cu") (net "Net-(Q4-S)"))
 (via (at 139.2 112.4) (size 0.9) (drill 0.4) (layers "F.Cu" "B.Cu") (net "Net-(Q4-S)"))
 (via (at 136 116.2) (size 0.9) (drill 0.4) (layers "F.Cu" "B.Cu") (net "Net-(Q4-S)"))
 (segment (start 139.2 113.6) (end 136.6 116.2) (width 0.4) (layer "B.Cu") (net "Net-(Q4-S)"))
 (segment (start 139.2 113.6) (end 139.5625 113.9625) (width 0.4) (layer "B.Cu") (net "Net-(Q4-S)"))
 (segment (start 150 113.9625) (end 146.8 113.9625) (width 0.4) (layer "B.Cu") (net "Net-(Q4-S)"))
 (segment (start 139.2 112.4) (end 139.2 113.6) (width 0.4) (layer "B.Cu") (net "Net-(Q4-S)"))
 (segment (start 139.5625 113.9625) (end 146.8 113.9625) (width 0.4) (layer "B.Cu") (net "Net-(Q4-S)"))
 (segment (start 136.6 116.2) (end 136 116.2) (width 0.4) (layer "B.Cu") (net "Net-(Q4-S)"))
 (segment (start 151.3 113.90855) (end 150.358549 114.850001) (width 0.4) (layer "F.Cu") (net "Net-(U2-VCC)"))
 (segment (start 149.7 108.2375) (end 151.3 109.8375) (width 0.4) (layer "F.Cu") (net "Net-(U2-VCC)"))
 (segment (start 145.3 109.5) (end 148.4375 109.5) (width 0.4) (layer "F.Cu") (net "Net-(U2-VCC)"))
 (segment (start 150.358549 114.850001) (end 149.69605 114.850001) (width 0.4) (layer "F.Cu") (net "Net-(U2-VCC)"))
 (segment (start 148.4375 109.5) (end 149.7 108.2375) (width 0.4) (layer "F.Cu") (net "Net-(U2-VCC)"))
 (segment (start 151.3 109.8375) (end 151.3 113.90855) (width 0.4) (layer "F.Cu") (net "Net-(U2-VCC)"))
 (segment (start 147.42105 114.850001) (end 148.083549 114.850001) (width 0.4) (layer "F.Cu") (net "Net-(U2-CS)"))
 (segment (start 148.63355 115.400002) (end 148.63355 116.93355) (width 0.4) (layer "F.Cu") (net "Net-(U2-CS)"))
 (segment (start 151.7 117.2) (end 152.8 116.1) (width 0.4) (layer "F.Cu") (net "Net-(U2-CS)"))
 (segment (start 152.8 116.1) (end 152.8 112.9) (width 0.4) (layer "F.Cu") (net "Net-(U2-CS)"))
 (segment (start 148.083549 114.850001) (end 148.63355 115.400002) (width 0.4) (layer "F.Cu") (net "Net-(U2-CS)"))
 (segment (start 148.9 117.2) (end 151.7 117.2) (width 0.4) (layer "F.Cu") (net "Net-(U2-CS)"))
 (segment (start 148.63355 116.93355) (end 148.9 117.2) (width 0.4) (layer "F.Cu") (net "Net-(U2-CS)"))
 (segment (start 144.333001 92.197499) (end 149.5505 86.98) (width 1) (layer "F.Cu") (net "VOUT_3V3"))
 (segment (start 150.748 86.917) (end 150.685 86.98) (width 0.4) (layer "F.Cu") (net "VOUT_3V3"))
 (segment (start 152.387501 102.187501) (end 143.287501 102.187501) (width 0.4) (layer "F.Cu") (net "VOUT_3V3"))
 (segment (start 143.287501 102.187501) (end 144.333001 101.142) (width 1) (layer "F.Cu") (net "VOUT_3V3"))
 (segment (start 144.333001 92.7) (end 144.333001 92.197499) (width 1) (layer "F.Cu") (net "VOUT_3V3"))
 (segment (start 153.753 100.822002) (end 152.387501 102.187501) (width 0.4) (layer "F.Cu") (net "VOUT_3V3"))
 (segment (start 134.05 112.1625) (end 134.05 111.425001) (width 1) (layer "F.Cu") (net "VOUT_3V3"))
 (segment (start 139.287501 106.187501) (end 143.287501 102.187501) (width 1) (layer "F.Cu") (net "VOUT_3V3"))
 (segment (start 144.233001 92.6) (end 144.333001 92.7) (width 0.4) (layer "F.Cu") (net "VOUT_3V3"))
 (segment (start 153.753 86.917) (end 150.748 86.917) (width 0.4) (layer "F.Cu") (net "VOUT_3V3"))
 (segment (start 153.753 97.077) (end 153.753 100.822002) (width 0.4) (layer "F.Cu") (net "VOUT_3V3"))
 (segment (start 134.05 111.425001) (end 139.287501 106.187501) (width 1) (layer "F.Cu") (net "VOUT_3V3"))
 (segment (start 142.7 92.6) (end 144.233001 92.6) (width 0.4) (layer "F.Cu") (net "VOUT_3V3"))
 (segment (start 144.333001 101.142) (end 144.333001 92.7) (width 1) (layer "F.Cu") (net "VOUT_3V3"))
 (segment (start 149.5505 86.98) (end 150.685 86.98) (width 1) (layer "F.Cu") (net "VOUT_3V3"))
 (via (at 134.3 106.2) (size 0.9) (drill 0.4) (layers "F.Cu" "B.Cu") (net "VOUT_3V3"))
 (via (at 142.7 92.6) (size 0.9) (drill 0.4) (layers "F.Cu" "B.Cu") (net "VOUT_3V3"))
 (via (at 139.287501 106.187501) (size 0.9) (drill 0.4) (layers "F.Cu" "B.Cu") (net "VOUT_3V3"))
 (segment (start 142.3 90.7625) (end 142.3 92.2) (width 0.4) (layer "B.Cu") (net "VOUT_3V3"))
 (segment (start 136.2 107.9375) (end 136.0375 107.9375) (width 0.2) (layer "B.Cu") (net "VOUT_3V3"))
 (segment (start 131.515 103.415) (end 134.3 106.2) (width 0.4) (layer "B.Cu") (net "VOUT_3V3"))
 (segment (start 138.7 106.775002) (end 139.287501 106.187501) (width 0.4) (layer "B.Cu") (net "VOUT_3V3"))
 (segment (start 138.7 107.9375) (end 138.7 106.775002) (width 0.4) (layer "B.Cu") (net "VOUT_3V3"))
 (segment (start 142.3 92.2) (end 142.7 92.6) (width 0.4) (layer "B.Cu") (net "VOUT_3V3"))
 (segment (start 136.0375 107.9375) (end 134.3 106.2) (width 0.2) (layer "B.Cu") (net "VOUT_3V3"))
 (segment (start 131.515 99.363) (end 131.515 103.415) (width 0.4) (layer "B.Cu") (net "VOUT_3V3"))
 (segment (start 138.6 82.2) (end 138.6 85.9695) (width 0.2) (layer "F.Cu") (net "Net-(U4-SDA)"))
 (segment (start 135.0495 89.52) (end 134.715 89.52) (width 0.2) (layer "F.Cu") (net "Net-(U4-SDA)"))
 (segment (start 133.738 89.52) (end 134.715 89.52) (width 0.4) (layer "F.Cu") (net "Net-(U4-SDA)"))
 (segment (start 138.6 85.9695) (end 135.0495 89.52) (width 0.2) (layer "F.Cu") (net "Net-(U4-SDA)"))
 (segment (start 131.515 91.743) (end 133.738 89.52) (width 0.4) (layer "F.Cu") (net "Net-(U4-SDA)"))
 (via (at 138.6 82.2) (size 0.9) (drill 0.4) (layers "F.Cu" "B.Cu") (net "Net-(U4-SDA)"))
 (segment (start 139.15 81.65) (end 138.6 82.2) (width 0.2) (layer "B.Cu") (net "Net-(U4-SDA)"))
 (segment (start 150.5 83.734314) (end 148.415686 81.65) (width 0.2) (layer "B.Cu") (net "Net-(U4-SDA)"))
 (segment (start 153.753 89.457) (end 150.5 86.204) (width 0.2) (layer "B.Cu") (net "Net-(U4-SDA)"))
 (segment (start 148.415686 81.65) (end 139.15 81.65) (width 0.2) (layer "B.Cu") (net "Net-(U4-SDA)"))
 (segment (start 150.5 86.204) (end 150.5 83.734314) (width 0.2) (layer "B.Cu") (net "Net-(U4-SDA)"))
 (segment (start 139.8 82.4) (end 139.8 87.3095) (width 0.2) (layer "F.Cu") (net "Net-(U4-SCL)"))
 (segment (start 131.515 94.283) (end 133.738 92.06) (width 0.4) (layer "F.Cu") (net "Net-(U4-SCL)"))
 (segment (start 139.8 87.3095) (end 135.0495 92.06) (width 0.2) (layer "F.Cu") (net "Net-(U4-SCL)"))
 (segment (start 133.738 92.06) (end 134.715 92.06) (width 0.4) (layer "F.Cu") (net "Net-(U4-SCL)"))
 (segment (start 135.0495 92.06) (end 134.715 92.06) (width 0.2) (layer "F.Cu") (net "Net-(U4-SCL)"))
 (via (at 139.8 82.4) (size 0.9) (drill 0.4) (layers "F.Cu" "B.Cu") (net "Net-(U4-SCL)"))
 (segment (start 153.753 91.997) (end 150.1 88.344) (width 0.2) (layer "B.Cu") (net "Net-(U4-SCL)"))
 (segment (start 148.6 82.4) (end 139.8 82.4) (width 0.2) (layer "B.Cu") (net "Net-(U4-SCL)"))
 (segment (start 150.1 88.344) (end 150.1 83.9) (width 0.2) (layer "B.Cu") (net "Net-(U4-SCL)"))
 (segment (start 150.1 83.9) (end 148.6 82.4) (width 0.2) (layer "B.Cu") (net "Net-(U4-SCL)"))
 (segment (start 138.3 94.6) (end 134.715 94.6) (width 0.4) (layer "F.Cu") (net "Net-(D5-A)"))
 (via (at 138.3 94.6) (size 0.9) (drill 0.4) (layers "F.Cu" "B.Cu") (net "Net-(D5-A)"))
 (segment (start 140.3125 94.6) (end 138.3 94.6) (width 0.4) (layer "B.Cu") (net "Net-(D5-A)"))
 (segment (start 144.4 98.2) (end 144.4 95.7125) (width 0.4) (layer "B.Cu") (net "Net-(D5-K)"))
 (segment (start 144.4 95.7125) (end 143.2875 94.6) (width 0.4) (layer "B.Cu") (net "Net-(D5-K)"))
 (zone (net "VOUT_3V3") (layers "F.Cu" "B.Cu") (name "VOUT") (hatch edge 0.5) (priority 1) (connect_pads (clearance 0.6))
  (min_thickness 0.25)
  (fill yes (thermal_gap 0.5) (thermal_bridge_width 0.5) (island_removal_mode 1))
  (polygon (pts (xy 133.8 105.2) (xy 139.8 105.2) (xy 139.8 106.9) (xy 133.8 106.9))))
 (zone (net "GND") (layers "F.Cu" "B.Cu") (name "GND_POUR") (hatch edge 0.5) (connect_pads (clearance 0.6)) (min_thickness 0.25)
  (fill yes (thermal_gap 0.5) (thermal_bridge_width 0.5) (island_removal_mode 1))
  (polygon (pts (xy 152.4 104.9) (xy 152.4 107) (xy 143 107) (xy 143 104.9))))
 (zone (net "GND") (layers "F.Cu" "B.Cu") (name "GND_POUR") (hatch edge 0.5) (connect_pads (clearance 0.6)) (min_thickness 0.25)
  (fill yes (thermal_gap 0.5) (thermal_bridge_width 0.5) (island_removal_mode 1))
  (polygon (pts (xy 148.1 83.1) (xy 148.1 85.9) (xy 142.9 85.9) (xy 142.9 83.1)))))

